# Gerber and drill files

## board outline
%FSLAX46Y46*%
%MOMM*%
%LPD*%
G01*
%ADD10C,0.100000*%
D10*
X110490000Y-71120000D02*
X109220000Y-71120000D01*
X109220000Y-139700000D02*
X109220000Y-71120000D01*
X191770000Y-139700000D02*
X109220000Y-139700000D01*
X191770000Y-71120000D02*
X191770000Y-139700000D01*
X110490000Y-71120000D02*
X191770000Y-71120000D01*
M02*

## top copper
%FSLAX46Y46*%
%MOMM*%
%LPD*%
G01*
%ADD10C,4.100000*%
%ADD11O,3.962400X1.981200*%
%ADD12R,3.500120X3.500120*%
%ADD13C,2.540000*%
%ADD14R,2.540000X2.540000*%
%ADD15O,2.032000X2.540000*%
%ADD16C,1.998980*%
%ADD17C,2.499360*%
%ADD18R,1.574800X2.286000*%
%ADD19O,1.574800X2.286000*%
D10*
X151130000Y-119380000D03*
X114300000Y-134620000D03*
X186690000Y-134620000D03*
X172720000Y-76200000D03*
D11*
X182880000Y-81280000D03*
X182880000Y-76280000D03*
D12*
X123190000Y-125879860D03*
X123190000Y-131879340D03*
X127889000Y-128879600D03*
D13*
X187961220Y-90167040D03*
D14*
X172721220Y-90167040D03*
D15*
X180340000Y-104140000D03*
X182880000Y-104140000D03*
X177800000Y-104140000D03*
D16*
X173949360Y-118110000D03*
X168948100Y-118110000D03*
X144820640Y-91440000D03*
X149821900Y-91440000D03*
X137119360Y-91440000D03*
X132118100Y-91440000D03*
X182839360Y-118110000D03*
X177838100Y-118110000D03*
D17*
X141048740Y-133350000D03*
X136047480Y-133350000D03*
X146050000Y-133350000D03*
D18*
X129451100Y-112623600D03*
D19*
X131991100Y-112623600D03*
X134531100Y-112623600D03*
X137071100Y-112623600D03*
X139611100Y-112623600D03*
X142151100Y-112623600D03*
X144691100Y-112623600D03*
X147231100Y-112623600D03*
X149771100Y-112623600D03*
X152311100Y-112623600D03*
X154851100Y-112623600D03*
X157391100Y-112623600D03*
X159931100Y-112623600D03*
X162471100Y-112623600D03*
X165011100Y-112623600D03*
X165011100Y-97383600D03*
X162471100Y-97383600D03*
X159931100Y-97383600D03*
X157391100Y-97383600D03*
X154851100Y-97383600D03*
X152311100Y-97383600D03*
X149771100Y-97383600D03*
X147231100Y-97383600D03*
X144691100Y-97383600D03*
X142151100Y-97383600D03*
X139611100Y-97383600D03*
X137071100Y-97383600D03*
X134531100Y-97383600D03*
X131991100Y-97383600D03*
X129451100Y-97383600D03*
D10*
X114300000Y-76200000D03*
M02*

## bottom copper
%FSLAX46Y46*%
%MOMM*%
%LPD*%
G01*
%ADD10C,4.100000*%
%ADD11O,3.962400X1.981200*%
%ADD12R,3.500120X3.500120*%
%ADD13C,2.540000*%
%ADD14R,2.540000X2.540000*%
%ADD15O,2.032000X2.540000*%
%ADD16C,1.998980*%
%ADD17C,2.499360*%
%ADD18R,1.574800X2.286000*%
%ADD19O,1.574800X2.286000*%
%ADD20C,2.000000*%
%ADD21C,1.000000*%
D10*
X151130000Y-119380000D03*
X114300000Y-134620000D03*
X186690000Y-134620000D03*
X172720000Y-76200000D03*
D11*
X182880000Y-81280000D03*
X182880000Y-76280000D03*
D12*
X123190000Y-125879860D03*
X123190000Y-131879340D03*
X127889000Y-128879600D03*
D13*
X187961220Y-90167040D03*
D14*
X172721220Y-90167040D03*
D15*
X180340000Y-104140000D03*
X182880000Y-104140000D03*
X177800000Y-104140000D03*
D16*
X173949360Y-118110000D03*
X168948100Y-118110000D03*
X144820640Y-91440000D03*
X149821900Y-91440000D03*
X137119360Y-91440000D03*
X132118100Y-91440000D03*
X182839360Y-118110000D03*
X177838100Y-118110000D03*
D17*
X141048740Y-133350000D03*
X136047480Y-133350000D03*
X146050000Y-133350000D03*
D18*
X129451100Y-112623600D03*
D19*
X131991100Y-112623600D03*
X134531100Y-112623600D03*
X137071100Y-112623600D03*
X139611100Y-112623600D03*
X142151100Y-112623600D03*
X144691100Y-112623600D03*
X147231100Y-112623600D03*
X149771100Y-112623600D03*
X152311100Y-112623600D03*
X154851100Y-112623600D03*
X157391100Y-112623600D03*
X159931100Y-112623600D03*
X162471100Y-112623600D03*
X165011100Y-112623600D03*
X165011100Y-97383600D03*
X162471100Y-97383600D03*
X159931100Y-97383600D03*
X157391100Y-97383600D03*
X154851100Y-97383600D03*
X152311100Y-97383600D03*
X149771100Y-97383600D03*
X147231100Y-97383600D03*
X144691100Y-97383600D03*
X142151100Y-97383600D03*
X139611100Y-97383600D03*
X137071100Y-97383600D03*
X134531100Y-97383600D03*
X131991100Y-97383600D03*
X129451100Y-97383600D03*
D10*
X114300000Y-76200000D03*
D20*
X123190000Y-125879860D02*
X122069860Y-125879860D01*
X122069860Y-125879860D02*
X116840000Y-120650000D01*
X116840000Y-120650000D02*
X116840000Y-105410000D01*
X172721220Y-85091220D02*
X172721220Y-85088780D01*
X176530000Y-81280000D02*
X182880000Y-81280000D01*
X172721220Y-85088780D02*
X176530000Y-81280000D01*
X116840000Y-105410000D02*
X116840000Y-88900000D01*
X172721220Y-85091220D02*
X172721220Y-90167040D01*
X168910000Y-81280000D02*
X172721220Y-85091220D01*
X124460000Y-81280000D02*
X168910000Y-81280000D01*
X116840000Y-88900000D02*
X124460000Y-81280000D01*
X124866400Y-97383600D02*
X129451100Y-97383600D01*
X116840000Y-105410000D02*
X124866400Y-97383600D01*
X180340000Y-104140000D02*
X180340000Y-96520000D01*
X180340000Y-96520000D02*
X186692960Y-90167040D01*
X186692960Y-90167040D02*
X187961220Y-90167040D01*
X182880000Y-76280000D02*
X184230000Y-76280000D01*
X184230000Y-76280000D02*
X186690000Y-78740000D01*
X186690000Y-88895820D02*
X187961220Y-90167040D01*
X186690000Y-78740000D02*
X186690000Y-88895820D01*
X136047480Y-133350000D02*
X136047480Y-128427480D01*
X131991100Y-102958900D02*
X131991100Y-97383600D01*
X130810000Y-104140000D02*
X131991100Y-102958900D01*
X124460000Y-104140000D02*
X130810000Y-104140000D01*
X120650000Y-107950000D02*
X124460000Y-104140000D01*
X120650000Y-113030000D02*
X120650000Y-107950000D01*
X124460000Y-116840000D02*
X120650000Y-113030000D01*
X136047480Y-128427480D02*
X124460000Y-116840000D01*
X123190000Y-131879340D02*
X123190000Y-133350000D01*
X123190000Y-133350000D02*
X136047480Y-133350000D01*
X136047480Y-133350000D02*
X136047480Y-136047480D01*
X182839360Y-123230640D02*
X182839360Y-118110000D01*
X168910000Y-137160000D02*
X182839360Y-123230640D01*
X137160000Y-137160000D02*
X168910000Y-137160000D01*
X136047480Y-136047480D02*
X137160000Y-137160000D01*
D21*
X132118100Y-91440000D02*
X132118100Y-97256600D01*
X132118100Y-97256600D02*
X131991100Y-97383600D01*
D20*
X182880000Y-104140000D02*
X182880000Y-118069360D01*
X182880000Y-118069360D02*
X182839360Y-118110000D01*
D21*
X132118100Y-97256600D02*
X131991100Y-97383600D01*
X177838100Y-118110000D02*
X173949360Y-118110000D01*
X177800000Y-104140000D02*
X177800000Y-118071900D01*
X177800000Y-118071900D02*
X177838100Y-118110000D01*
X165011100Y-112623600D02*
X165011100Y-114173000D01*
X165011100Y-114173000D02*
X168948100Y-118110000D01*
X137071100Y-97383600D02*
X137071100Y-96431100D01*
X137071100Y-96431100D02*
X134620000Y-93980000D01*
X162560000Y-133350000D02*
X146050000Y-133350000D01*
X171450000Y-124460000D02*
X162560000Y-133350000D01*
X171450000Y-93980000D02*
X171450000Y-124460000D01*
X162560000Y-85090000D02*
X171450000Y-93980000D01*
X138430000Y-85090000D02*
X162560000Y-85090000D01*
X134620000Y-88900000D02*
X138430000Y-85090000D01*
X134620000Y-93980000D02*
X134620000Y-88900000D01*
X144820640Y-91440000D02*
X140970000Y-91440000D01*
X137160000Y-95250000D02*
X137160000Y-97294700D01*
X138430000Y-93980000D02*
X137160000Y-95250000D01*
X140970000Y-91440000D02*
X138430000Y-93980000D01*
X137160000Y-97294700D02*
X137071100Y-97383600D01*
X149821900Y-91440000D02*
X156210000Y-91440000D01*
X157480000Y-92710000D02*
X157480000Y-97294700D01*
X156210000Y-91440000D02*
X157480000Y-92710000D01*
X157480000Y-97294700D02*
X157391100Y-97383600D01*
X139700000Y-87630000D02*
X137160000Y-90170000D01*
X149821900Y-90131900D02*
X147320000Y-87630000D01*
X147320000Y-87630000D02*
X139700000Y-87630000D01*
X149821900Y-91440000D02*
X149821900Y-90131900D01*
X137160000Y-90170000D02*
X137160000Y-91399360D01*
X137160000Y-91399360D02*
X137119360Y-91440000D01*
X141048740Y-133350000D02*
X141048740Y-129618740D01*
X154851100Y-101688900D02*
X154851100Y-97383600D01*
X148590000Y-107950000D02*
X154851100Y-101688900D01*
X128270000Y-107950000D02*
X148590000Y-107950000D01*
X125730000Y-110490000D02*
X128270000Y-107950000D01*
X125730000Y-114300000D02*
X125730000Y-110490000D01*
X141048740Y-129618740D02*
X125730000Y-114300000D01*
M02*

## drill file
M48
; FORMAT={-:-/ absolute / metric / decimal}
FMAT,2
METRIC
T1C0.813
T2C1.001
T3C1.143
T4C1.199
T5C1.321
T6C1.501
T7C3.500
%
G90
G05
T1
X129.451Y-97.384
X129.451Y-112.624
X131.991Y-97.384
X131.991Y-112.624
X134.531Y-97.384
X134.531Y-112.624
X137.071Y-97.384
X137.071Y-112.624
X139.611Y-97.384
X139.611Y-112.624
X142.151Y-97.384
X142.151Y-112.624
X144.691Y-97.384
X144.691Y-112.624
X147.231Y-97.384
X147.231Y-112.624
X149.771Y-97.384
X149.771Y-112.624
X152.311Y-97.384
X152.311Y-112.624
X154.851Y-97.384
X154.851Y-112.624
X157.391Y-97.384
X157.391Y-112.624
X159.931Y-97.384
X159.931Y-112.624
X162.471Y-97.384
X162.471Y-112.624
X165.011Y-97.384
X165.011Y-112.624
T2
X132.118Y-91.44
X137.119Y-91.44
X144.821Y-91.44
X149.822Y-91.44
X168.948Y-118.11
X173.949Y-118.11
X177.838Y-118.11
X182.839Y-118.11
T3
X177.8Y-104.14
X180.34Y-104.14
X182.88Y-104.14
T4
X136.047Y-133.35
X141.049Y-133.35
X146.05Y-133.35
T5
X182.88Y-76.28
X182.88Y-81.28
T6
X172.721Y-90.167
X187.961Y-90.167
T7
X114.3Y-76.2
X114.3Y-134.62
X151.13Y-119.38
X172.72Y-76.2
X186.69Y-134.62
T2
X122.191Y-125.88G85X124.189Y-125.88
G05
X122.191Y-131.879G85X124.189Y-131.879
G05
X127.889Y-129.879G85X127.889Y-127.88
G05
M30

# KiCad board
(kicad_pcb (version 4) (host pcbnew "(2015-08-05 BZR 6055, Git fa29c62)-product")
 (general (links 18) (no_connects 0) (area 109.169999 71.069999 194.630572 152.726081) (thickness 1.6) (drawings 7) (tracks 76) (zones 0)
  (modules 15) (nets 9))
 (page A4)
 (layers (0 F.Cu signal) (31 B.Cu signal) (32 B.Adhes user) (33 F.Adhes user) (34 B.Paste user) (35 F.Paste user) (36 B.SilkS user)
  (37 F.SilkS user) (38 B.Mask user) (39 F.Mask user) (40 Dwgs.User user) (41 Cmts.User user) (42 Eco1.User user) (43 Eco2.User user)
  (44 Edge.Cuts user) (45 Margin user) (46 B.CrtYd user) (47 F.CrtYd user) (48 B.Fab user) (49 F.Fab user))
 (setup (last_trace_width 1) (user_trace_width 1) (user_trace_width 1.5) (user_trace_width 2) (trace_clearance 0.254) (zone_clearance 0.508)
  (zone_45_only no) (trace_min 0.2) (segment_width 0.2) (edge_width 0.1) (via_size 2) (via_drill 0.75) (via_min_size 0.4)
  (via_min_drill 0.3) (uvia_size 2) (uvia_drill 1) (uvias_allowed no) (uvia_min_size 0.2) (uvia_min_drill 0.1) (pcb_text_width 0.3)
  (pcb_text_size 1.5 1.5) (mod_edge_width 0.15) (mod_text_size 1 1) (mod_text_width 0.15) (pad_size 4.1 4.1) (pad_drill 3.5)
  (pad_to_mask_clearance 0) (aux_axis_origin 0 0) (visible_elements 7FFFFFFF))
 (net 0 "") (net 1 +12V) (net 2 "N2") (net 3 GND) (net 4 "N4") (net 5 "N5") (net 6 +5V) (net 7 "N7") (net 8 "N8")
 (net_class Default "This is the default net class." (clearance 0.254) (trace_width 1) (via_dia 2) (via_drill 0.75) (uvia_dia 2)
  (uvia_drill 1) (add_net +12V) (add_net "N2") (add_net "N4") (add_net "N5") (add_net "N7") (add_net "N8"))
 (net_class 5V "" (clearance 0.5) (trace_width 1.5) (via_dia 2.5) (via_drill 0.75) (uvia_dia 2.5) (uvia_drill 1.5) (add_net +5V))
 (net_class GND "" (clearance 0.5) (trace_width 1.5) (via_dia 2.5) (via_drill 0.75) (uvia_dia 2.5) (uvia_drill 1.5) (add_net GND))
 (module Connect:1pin (layer F.Cu) (at 151.13 119.38)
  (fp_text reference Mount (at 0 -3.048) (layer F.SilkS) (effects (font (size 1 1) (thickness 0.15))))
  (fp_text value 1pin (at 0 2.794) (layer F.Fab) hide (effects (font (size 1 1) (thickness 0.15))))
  (pad 1 thru_hole circle (at 0 0) (size 4.1 4.1) (drill 3.5) (layers *.Cu *.Mask F.SilkS)))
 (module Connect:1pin (layer F.Cu) (at 114.3 134.62)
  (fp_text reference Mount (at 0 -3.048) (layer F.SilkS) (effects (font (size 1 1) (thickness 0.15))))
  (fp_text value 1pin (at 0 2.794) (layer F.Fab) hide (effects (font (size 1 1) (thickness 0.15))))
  (pad 1 thru_hole circle (at 0 0) (size 4.1 4.1) (drill 3.5) (layers *.Cu *.Mask F.SilkS)))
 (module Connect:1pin (layer F.Cu) (at 186.69 134.62)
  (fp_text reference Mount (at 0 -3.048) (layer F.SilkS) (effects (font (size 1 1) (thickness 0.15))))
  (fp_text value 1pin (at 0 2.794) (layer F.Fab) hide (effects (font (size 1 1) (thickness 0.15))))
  (pad 1 thru_hole circle (at 0 0) (size 4.1 4.1) (drill 3.5) (layers *.Cu *.Mask F.SilkS)))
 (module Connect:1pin (layer F.Cu) (at 172.72 76.2)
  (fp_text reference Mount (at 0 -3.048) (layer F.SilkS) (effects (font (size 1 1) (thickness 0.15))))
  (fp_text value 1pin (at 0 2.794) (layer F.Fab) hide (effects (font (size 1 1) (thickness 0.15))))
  (pad 1 thru_hole circle (at 0 0) (size 4.1 4.1) (drill 3.5) (layers *.Cu *.Mask F.SilkS)))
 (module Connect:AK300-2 (layer F.Cu) (at 182.88 81.28 90)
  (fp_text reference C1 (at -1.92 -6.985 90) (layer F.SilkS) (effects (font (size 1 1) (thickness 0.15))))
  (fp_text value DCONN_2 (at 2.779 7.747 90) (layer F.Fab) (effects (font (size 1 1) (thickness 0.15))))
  (pad 1 thru_hole oval (at 0 0 90) (size 1.9812 3.9624) (drill 1.3208) (layers *.Cu F.Paste F.SilkS F.Mask) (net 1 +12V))
  (pad 2 thru_hole oval (at 5 0 90) (size 1.9812 3.9624) (drill 1.3208) (layers *.Cu F.Paste F.SilkS F.Mask) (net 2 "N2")))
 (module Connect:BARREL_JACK (layer F.Cu) (at 123.19 132.08 90)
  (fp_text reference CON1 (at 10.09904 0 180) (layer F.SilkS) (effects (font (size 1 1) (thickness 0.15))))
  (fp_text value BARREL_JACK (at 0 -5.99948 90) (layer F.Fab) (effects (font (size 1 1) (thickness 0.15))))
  (pad 1 thru_hole rect (at 6.20014 0 90) (size 3.50012 3.50012) (drill oval 1.00076 2.99974) (layers *.Cu *.Mask F.SilkS) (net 1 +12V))
  (pad 2 thru_hole rect (at 0.20066 0 90) (size 3.50012 3.50012) (drill oval 1.00076 2.99974) (layers *.Cu *.Mask F.SilkS) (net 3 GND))
  (pad 3 thru_hole rect (at 3.2004 4.699 90) (size 3.50012 3.50012) (drill oval 2.99974 1.00076) (layers *.Cu *.Mask F.SilkS)))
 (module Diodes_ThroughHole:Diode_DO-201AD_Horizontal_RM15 (layer F.Cu) (at 172.72 90.17)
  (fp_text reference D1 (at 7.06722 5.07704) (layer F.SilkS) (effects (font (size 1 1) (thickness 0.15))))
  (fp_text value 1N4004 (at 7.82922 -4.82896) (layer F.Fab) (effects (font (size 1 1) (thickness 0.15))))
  (pad 2 thru_hole circle (at 15.24122 -0.00296 180) (size 2.54 2.54) (drill 1.50114) (layers *.Cu *.Mask F.SilkS) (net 2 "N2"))
  (pad 1 thru_hole rect (at 0.00122 -0.00296 180) (size 2.54 2.54) (drill 1.50114) (layers *.Cu *.Mask F.SilkS) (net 1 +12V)))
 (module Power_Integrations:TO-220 (layer F.Cu) (at 180.34 104.14)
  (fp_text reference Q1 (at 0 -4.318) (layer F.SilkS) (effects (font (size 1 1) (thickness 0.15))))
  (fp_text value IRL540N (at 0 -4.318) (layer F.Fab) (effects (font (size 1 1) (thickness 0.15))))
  (pad 2 thru_hole oval (at 0 0) (size 2.032 2.54) (drill 1.143) (layers *.Cu *.Mask F.SilkS) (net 2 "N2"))
  (pad 3 thru_hole oval (at 2.54 0) (size 2.032 2.54) (drill 1.143) (layers *.Cu *.Mask F.SilkS) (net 3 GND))
  (pad 1 thru_hole oval (at -2.54 0) (size 2.032 2.54) (drill 1.143) (layers *.Cu *.Mask F.SilkS) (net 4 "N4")))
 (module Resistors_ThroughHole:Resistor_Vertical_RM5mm (layer F.Cu) (at 171.45 118.11 180)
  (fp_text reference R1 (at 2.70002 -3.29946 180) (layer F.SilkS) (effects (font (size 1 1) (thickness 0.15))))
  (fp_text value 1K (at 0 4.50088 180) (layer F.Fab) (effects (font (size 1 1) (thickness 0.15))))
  (pad 1 thru_hole circle (at -2.49936 0 180) (size 1.99898 1.99898) (drill 1.00076) (layers *.Cu *.SilkS *.Mask) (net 4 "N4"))
  (pad 2 thru_hole circle (at 2.5019 0 180) (size 1.99898 1.99898) (drill 1.00076) (layers *.Cu *.SilkS *.Mask) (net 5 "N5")))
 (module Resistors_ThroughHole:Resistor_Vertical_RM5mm (layer F.Cu) (at 147.32 91.44)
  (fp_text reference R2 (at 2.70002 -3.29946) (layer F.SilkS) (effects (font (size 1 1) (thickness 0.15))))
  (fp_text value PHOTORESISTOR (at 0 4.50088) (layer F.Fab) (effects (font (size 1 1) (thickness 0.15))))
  (pad 1 thru_hole circle (at -2.49936 0) (size 1.99898 1.99898) (drill 1.00076) (layers *.Cu *.SilkS *.Mask) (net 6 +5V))
  (pad 2 thru_hole circle (at 2.5019 0) (size 1.99898 1.99898) (drill 1.00076) (layers *.Cu *.SilkS *.Mask) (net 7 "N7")))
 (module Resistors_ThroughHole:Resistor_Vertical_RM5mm (layer F.Cu) (at 134.62 91.44 180)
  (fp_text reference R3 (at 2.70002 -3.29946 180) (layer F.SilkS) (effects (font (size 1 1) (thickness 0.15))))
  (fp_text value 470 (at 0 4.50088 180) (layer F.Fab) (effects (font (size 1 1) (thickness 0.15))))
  (pad 1 thru_hole circle (at -2.49936 0 180) (size 1.99898 1.99898) (drill 1.00076) (layers *.Cu *.SilkS *.Mask) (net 7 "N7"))
  (pad 2 thru_hole circle (at 2.5019 0 180) (size 1.99898 1.99898) (drill 1.00076) (layers *.Cu *.SilkS *.Mask) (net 3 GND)))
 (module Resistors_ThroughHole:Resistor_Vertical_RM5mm (layer F.Cu) (at 180.34 118.11 180)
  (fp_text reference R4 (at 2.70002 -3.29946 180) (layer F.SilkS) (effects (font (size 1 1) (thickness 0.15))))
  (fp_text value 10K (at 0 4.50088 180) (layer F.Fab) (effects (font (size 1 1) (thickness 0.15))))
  (pad 1 thru_hole circle (at -2.49936 0 180) (size 1.99898 1.99898) (drill 1.00076) (layers *.Cu *.SilkS *.Mask) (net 3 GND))
  (pad 2 thru_hole circle (at 2.5019 0 180) (size 1.99898 1.99898) (drill 1.00076) (layers *.Cu *.SilkS *.Mask) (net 4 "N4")))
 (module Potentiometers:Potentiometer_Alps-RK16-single (layer F.Cu) (at 146.05 133.35 270)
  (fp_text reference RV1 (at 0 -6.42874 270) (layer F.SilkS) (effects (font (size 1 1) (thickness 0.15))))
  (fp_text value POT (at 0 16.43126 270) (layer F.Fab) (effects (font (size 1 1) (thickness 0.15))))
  (pad 2 thru_hole circle (at 0 5.00126 270) (size 2.49936 2.49936) (drill 1.19888) (layers *.Cu *.Mask F.SilkS) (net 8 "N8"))
  (pad 3 thru_hole circle (at 0 10.00252 270) (size 2.49936 2.49936) (drill 1.19888) (layers *.Cu *.Mask F.SilkS) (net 3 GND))
  (pad 1 thru_hole circle (at 0 0 270) (size 2.49936 2.49936) (drill 1.19888) (layers *.Cu *.Mask F.SilkS) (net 6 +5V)))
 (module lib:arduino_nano (layer F.Cu) (at 148.5011 105.0036)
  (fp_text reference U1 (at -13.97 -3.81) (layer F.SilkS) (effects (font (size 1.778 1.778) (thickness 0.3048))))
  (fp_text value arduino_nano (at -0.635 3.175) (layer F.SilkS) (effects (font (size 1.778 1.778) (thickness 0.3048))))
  (pad TX1 thru_hole rect (at -19.05 7.62) (size 1.5748 2.286) (drill 0.8128) (layers *.Cu *.Mask F.SilkS))
  (pad RX0 thru_hole oval (at -16.51 7.62) (size 1.5748 2.286) (drill 0.8128) (layers *.Cu *.Mask F.SilkS))
  (pad RST1 thru_hole oval (at -13.97 7.62) (size 1.5748 2.286) (drill 0.8128) (layers *.Cu *.Mask F.SilkS))
  (pad GND1 thru_hole oval (at -11.43 7.62) (size 1.5748 2.286) (drill 0.8128) (layers *.Cu *.Mask F.SilkS))
  (pad D2 thru_hole oval (at -8.89 7.62) (size 1.5748 2.286) (drill 0.8128) (layers *.Cu *.Mask F.SilkS))
  (pad D3 thru_hole oval (at -6.35 7.62) (size 1.5748 2.286) (drill 0.8128) (layers *.Cu *.Mask F.SilkS))
  (pad D4 thru_hole oval (at -3.81 7.62) (size 1.5748 2.286) (drill 0.8128) (layers *.Cu *.Mask F.SilkS))
  (pad D5 thru_hole oval (at -1.27 7.62) (size 1.5748 2.286) (drill 0.8128) (layers *.Cu *.Mask F.SilkS))
  (pad D6 thru_hole oval (at 1.27 7.62) (size 1.5748 2.286) (drill 0.8128) (layers *.Cu *.Mask F.SilkS))
  (pad D7 thru_hole oval (at 3.81 7.62) (size 1.5748 2.286) (drill 0.8128) (layers *.Cu *.Mask F.SilkS))
  (pad D8 thru_hole oval (at 6.35 7.62) (size 1.5748 2.286) (drill 0.8128) (layers *.Cu *.Mask F.SilkS))
  (pad D9 thru_hole oval (at 8.89 7.62) (size 1.5748 2.286) (drill 0.8128) (layers *.Cu *.Mask F.SilkS))
  (pad D10 thru_hole oval (at 11.43 7.62) (size 1.5748 2.286) (drill 0.8128) (layers *.Cu *.Mask F.SilkS))
  (pad D11 thru_hole oval (at 13.97 7.62) (size 1.5748 2.286) (drill 0.8128) (layers *.Cu *.Mask F.SilkS))
  (pad D12 thru_hole oval (at 16.51 7.62) (size 1.5748 2.286) (drill 0.8128) (layers *.Cu *.Mask F.SilkS) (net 5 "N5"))
  (pad D13 thru_hole oval (at 16.51 -7.62) (size 1.5748 2.286) (drill 0.8128) (layers *.Cu *.Mask F.SilkS))
  (pad 3V3 thru_hole oval (at 13.97 -7.62) (size 1.5748 2.286) (drill 0.8128) (layers *.Cu *.Mask F.SilkS))
  (pad REF thru_hole oval (at 11.43 -7.62) (size 1.5748 2.286) (drill 0.8128) (layers *.Cu *.Mask F.SilkS))
  (pad A0 thru_hole oval (at 8.89 -7.62) (size 1.5748 2.286) (drill 0.8128) (layers *.Cu *.Mask F.SilkS) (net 7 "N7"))
  (pad A1 thru_hole oval (at 6.35 -7.62) (size 1.5748 2.286) (drill 0.8128) (layers *.Cu *.Mask F.SilkS) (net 8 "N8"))
  (pad A2 thru_hole oval (at 3.81 -7.62) (size 1.5748 2.286) (drill 0.8128) (layers *.Cu *.Mask F.SilkS))
  (pad A3 thru_hole oval (at 1.27 -7.62) (size 1.5748 2.286) (drill 0.8128) (layers *.Cu *.Mask F.SilkS))
  (pad A4 thru_hole oval (at -1.27 -7.62) (size 1.5748 2.286) (drill 0.8128) (layers *.Cu *.Mask F.SilkS))
  (pad A5 thru_hole oval (at -3.81 -7.62) (size 1.5748 2.286) (drill 0.8128) (layers *.Cu *.Mask F.SilkS))
  (pad A6 thru_hole oval (at -6.35 -7.62) (size 1.5748 2.286) (drill 0.8128) (layers *.Cu *.Mask F.SilkS))
  (pad A7 thru_hole oval (at -8.89 -7.62) (size 1.5748 2.286) (drill 0.8128) (layers *.Cu *.Mask F.SilkS))
  (pad 5V thru_hole oval (at -11.43 -7.62) (size 1.5748 2.286) (drill 0.8128) (layers *.Cu *.Mask F.SilkS) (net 6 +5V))
  (pad RST thru_hole oval (at -13.97 -7.62) (size 1.5748 2.286) (drill 0.8128) (layers *.Cu *.Mask F.SilkS))
  (pad GND thru_hole oval (at -16.51 -7.62) (size 1.5748 2.286) (drill 0.8128) (layers *.Cu *.Mask F.SilkS) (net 3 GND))
  (pad VIN thru_hole oval (at -19.05 -7.62) (size 1.5748 2.286) (drill 0.8128) (layers *.Cu *.Mask F.SilkS) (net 1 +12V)))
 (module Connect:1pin (layer F.Cu) (at 114.3 76.2)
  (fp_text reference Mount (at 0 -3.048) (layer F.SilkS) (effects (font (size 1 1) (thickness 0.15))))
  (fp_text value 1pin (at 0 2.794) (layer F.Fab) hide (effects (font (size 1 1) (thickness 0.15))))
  (pad 1 thru_hole circle (at 0 0) (size 4.1 4.1) (drill 3.5) (layers *.Cu *.Mask F.SilkS)))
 (gr_line (start 110.49 71.12) (end 109.22 71.12) (angle 90) (layer Edge.Cuts) (width 0.1))
 (gr_line (start 109.22 139.7) (end 109.22 71.12) (angle 90) (layer Edge.Cuts) (width 0.1))
 (gr_line (start 191.77 139.7) (end 109.22 139.7) (angle 90) (layer Edge.Cuts) (width 0.1))
 (gr_line (start 191.77 71.12) (end 191.77 139.7) (angle 90) (layer Edge.Cuts) (width 0.1))
 (gr_line (start 110.49 71.12) (end 191.77 71.12) (angle 90) (layer Edge.Cuts) (width 0.1))
 (segment (start 123.19 125.87986) (end 122.06986 125.87986) (width 2) (layer B.Cu) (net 1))
 (segment (start 122.06986 125.87986) (end 116.84 120.65) (width 2) (layer B.Cu) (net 1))
 (segment (start 116.84 120.65) (end 116.84 105.41) (width 2) (layer B.Cu) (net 1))
 (segment (start 172.72122 85.09122) (end 172.72122 85.08878) (width 2) (layer B.Cu) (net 1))
 (segment (start 176.53 81.28) (end 182.88 81.28) (width 2) (layer B.Cu) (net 1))
 (segment (start 172.72122 85.08878) (end 176.53 81.28) (width 2) (layer B.Cu) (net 1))
 (segment (start 116.84 105.41) (end 116.84 88.9) (width 2) (layer B.Cu) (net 1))
 (segment (start 172.72122 85.09122) (end 172.72122 90.16704) (width 2) (layer B.Cu) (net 1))
 (segment (start 168.91 81.28) (end 172.72122 85.09122) (width 2) (layer B.Cu) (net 1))
 (segment (start 124.46 81.28) (end 168.91 81.28) (width 2) (layer B.Cu) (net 1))
 (segment (start 116.84 88.9) (end 124.46 81.28) (width 2) (layer B.Cu) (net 1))
 (segment (start 124.8664 97.3836) (end 129.4511 97.3836) (width 2) (layer B.Cu) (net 1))
 (segment (start 116.84 105.41) (end 124.8664 97.3836) (width 2) (layer B.Cu) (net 1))
 (segment (start 180.34 104.14) (end 180.34 96.52) (width 2) (layer B.Cu) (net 2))
 (segment (start 180.34 96.52) (end 186.69296 90.16704) (width 2) (layer B.Cu) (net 2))
 (segment (start 186.69296 90.16704) (end 187.96122 90.16704) (width 2) (layer B.Cu) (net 2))
 (segment (start 182.88 76.28) (end 184.23 76.28) (width 2) (layer B.Cu) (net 2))
 (segment (start 184.23 76.28) (end 186.69 78.74) (width 2) (layer B.Cu) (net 2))
 (segment (start 186.69 88.89582) (end 187.96122 90.16704) (width 2) (layer B.Cu) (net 2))
 (segment (start 186.69 78.74) (end 186.69 88.89582) (width 2) (layer B.Cu) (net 2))
 (segment (start 136.04748 133.35) (end 136.04748 128.42748) (width 2) (layer B.Cu) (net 3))
 (segment (start 131.9911 102.9589) (end 131.9911 97.3836) (width 2) (layer B.Cu) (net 3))
 (segment (start 130.81 104.14) (end 131.9911 102.9589) (width 2) (layer B.Cu) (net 3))
 (segment (start 124.46 104.14) (end 130.81 104.14) (width 2) (layer B.Cu) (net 3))
 (segment (start 120.65 107.95) (end 124.46 104.14) (width 2) (layer B.Cu) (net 3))
 (segment (start 120.65 113.03) (end 120.65 107.95) (width 2) (layer B.Cu) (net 3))
 (segment (start 124.46 116.84) (end 120.65 113.03) (width 2) (layer B.Cu) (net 3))
 (segment (start 136.04748 128.42748) (end 124.46 116.84) (width 2) (layer B.Cu) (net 3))
 (segment (start 123.19 131.87934) (end 123.19 133.35) (width 2) (layer B.Cu) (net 3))
 (segment (start 123.19 133.35) (end 136.04748 133.35) (width 2) (layer B.Cu) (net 3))
 (segment (start 136.04748 133.35) (end 136.04748 136.04748) (width 2) (layer B.Cu) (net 3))
 (segment (start 182.83936 123.23064) (end 182.83936 118.11) (width 2) (layer B.Cu) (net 3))
 (segment (start 168.91 137.16) (end 182.83936 123.23064) (width 2) (layer B.Cu) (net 3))
 (segment (start 137.16 137.16) (end 168.91 137.16) (width 2) (layer B.Cu) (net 3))
 (segment (start 136.04748 136.04748) (end 137.16 137.16) (width 2) (layer B.Cu) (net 3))
 (segment (start 132.1181 91.44) (end 132.1181 97.2566) (width 1) (layer B.Cu) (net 3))
 (segment (start 132.1181 97.2566) (end 131.9911 97.3836) (width 1) (layer B.Cu) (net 3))
 (segment (start 182.88 104.14) (end 182.88 118.06936) (width 2) (layer B.Cu) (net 3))
 (segment (start 182.88 118.06936) (end 182.83936 118.11) (width 2) (layer B.Cu) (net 3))
 (segment (start 132.1181 97.2566) (end 131.9911 97.3836) (width 1) (layer B.Cu) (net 3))
 (segment (start 177.8381 118.11) (end 173.94936 118.11) (width 1) (layer B.Cu) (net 4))
 (segment (start 177.8 104.14) (end 177.8 118.0719) (width 1) (layer B.Cu) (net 4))
 (segment (start 177.8 118.0719) (end 177.8381 118.11) (width 1) (layer B.Cu) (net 4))
 (segment (start 165.0111 112.6236) (end 165.0111 114.173) (width 1) (layer B.Cu) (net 5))
 (segment (start 165.0111 114.173) (end 168.9481 118.11) (width 1) (layer B.Cu) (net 5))
 (segment (start 137.0711 97.3836) (end 137.0711 96.4311) (width 1) (layer B.Cu) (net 6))
 (segment (start 137.0711 96.4311) (end 134.62 93.98) (width 1) (layer B.Cu) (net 6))
 (segment (start 162.56 133.35) (end 146.05 133.35) (width 1) (layer B.Cu) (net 6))
 (segment (start 171.45 124.46) (end 162.56 133.35) (width 1) (layer B.Cu) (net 6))
 (segment (start 171.45 93.98) (end 171.45 124.46) (width 1) (layer B.Cu) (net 6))
 (segment (start 162.56 85.09) (end 171.45 93.98) (width 1) (layer B.Cu) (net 6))
 (segment (start 138.43 85.09) (end 162.56 85.09) (width 1) (layer B.Cu) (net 6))
 (segment (start 134.62 88.9) (end 138.43 85.09) (width 1) (layer B.Cu) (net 6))
 (segment (start 134.62 93.98) (end 134.62 88.9) (width 1) (layer B.Cu) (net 6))
 (segment (start 144.82064 91.44) (end 140.97 91.44) (width 1) (layer B.Cu) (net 6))
 (segment (start 137.16 95.25) (end 137.16 97.2947) (width 1) (layer B.Cu) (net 6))
 (segment (start 138.43 93.98) (end 137.16 95.25) (width 1) (layer B.Cu) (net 6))
 (segment (start 140.97 91.44) (end 138.43 93.98) (width 1) (layer B.Cu) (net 6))
 (segment (start 137.16 97.2947) (end 137.0711 97.3836) (width 1) (layer B.Cu) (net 6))
 (segment (start 149.8219 91.44) (end 156.21 91.44) (width 1) (layer B.Cu) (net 7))
 (segment (start 157.48 92.71) (end 157.48 97.2947) (width 1) (layer B.Cu) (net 7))
 (segment (start 156.21 91.44) (end 157.48 92.71) (width 1) (layer B.Cu) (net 7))
 (segment (start 157.48 97.2947) (end 157.3911 97.3836) (width 1) (layer B.Cu) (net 7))
 (segment (start 139.7 87.63) (end 137.16 90.17) (width 1) (layer B.Cu) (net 7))
 (segment (start 149.8219 90.1319) (end 147.32 87.63) (width 1) (layer B.Cu) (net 7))
 (segment (start 147.32 87.63) (end 139.7 87.63) (width 1) (layer B.Cu) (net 7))
 (segment (start 149.8219 91.44) (end 149.8219 90.1319) (width 1) (layer B.Cu) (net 7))
 (segment (start 137.16 90.17) (end 137.16 91.39936) (width 1) (layer B.Cu) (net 7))
 (segment (start 137.16 91.39936) (end 137.11936 91.44) (width 1) (layer B.Cu) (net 7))
 (segment (start 141.04874 133.35) (end 141.04874 129.61874) (width 1) (layer B.Cu) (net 8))
 (segment (start 154.8511 101.6889) (end 154.8511 97.3836) (width 1) (layer B.Cu) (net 8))
 (segment (start 148.59 107.95) (end 154.8511 101.6889) (width 1) (layer B.Cu) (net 8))
 (segment (start 128.27 107.95) (end 148.59 107.95) (width 1) (layer B.Cu) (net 8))
 (segment (start 125.73 110.49) (end 128.27 107.95) (width 1) (layer B.Cu) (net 8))
 (segment (start 125.73 114.3) (end 125.73 110.49) (width 1) (layer B.Cu) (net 8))
 (segment (start 141.04874 129.61874) (end 125.73 114.3) (width 1) (layer B.Cu) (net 8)))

